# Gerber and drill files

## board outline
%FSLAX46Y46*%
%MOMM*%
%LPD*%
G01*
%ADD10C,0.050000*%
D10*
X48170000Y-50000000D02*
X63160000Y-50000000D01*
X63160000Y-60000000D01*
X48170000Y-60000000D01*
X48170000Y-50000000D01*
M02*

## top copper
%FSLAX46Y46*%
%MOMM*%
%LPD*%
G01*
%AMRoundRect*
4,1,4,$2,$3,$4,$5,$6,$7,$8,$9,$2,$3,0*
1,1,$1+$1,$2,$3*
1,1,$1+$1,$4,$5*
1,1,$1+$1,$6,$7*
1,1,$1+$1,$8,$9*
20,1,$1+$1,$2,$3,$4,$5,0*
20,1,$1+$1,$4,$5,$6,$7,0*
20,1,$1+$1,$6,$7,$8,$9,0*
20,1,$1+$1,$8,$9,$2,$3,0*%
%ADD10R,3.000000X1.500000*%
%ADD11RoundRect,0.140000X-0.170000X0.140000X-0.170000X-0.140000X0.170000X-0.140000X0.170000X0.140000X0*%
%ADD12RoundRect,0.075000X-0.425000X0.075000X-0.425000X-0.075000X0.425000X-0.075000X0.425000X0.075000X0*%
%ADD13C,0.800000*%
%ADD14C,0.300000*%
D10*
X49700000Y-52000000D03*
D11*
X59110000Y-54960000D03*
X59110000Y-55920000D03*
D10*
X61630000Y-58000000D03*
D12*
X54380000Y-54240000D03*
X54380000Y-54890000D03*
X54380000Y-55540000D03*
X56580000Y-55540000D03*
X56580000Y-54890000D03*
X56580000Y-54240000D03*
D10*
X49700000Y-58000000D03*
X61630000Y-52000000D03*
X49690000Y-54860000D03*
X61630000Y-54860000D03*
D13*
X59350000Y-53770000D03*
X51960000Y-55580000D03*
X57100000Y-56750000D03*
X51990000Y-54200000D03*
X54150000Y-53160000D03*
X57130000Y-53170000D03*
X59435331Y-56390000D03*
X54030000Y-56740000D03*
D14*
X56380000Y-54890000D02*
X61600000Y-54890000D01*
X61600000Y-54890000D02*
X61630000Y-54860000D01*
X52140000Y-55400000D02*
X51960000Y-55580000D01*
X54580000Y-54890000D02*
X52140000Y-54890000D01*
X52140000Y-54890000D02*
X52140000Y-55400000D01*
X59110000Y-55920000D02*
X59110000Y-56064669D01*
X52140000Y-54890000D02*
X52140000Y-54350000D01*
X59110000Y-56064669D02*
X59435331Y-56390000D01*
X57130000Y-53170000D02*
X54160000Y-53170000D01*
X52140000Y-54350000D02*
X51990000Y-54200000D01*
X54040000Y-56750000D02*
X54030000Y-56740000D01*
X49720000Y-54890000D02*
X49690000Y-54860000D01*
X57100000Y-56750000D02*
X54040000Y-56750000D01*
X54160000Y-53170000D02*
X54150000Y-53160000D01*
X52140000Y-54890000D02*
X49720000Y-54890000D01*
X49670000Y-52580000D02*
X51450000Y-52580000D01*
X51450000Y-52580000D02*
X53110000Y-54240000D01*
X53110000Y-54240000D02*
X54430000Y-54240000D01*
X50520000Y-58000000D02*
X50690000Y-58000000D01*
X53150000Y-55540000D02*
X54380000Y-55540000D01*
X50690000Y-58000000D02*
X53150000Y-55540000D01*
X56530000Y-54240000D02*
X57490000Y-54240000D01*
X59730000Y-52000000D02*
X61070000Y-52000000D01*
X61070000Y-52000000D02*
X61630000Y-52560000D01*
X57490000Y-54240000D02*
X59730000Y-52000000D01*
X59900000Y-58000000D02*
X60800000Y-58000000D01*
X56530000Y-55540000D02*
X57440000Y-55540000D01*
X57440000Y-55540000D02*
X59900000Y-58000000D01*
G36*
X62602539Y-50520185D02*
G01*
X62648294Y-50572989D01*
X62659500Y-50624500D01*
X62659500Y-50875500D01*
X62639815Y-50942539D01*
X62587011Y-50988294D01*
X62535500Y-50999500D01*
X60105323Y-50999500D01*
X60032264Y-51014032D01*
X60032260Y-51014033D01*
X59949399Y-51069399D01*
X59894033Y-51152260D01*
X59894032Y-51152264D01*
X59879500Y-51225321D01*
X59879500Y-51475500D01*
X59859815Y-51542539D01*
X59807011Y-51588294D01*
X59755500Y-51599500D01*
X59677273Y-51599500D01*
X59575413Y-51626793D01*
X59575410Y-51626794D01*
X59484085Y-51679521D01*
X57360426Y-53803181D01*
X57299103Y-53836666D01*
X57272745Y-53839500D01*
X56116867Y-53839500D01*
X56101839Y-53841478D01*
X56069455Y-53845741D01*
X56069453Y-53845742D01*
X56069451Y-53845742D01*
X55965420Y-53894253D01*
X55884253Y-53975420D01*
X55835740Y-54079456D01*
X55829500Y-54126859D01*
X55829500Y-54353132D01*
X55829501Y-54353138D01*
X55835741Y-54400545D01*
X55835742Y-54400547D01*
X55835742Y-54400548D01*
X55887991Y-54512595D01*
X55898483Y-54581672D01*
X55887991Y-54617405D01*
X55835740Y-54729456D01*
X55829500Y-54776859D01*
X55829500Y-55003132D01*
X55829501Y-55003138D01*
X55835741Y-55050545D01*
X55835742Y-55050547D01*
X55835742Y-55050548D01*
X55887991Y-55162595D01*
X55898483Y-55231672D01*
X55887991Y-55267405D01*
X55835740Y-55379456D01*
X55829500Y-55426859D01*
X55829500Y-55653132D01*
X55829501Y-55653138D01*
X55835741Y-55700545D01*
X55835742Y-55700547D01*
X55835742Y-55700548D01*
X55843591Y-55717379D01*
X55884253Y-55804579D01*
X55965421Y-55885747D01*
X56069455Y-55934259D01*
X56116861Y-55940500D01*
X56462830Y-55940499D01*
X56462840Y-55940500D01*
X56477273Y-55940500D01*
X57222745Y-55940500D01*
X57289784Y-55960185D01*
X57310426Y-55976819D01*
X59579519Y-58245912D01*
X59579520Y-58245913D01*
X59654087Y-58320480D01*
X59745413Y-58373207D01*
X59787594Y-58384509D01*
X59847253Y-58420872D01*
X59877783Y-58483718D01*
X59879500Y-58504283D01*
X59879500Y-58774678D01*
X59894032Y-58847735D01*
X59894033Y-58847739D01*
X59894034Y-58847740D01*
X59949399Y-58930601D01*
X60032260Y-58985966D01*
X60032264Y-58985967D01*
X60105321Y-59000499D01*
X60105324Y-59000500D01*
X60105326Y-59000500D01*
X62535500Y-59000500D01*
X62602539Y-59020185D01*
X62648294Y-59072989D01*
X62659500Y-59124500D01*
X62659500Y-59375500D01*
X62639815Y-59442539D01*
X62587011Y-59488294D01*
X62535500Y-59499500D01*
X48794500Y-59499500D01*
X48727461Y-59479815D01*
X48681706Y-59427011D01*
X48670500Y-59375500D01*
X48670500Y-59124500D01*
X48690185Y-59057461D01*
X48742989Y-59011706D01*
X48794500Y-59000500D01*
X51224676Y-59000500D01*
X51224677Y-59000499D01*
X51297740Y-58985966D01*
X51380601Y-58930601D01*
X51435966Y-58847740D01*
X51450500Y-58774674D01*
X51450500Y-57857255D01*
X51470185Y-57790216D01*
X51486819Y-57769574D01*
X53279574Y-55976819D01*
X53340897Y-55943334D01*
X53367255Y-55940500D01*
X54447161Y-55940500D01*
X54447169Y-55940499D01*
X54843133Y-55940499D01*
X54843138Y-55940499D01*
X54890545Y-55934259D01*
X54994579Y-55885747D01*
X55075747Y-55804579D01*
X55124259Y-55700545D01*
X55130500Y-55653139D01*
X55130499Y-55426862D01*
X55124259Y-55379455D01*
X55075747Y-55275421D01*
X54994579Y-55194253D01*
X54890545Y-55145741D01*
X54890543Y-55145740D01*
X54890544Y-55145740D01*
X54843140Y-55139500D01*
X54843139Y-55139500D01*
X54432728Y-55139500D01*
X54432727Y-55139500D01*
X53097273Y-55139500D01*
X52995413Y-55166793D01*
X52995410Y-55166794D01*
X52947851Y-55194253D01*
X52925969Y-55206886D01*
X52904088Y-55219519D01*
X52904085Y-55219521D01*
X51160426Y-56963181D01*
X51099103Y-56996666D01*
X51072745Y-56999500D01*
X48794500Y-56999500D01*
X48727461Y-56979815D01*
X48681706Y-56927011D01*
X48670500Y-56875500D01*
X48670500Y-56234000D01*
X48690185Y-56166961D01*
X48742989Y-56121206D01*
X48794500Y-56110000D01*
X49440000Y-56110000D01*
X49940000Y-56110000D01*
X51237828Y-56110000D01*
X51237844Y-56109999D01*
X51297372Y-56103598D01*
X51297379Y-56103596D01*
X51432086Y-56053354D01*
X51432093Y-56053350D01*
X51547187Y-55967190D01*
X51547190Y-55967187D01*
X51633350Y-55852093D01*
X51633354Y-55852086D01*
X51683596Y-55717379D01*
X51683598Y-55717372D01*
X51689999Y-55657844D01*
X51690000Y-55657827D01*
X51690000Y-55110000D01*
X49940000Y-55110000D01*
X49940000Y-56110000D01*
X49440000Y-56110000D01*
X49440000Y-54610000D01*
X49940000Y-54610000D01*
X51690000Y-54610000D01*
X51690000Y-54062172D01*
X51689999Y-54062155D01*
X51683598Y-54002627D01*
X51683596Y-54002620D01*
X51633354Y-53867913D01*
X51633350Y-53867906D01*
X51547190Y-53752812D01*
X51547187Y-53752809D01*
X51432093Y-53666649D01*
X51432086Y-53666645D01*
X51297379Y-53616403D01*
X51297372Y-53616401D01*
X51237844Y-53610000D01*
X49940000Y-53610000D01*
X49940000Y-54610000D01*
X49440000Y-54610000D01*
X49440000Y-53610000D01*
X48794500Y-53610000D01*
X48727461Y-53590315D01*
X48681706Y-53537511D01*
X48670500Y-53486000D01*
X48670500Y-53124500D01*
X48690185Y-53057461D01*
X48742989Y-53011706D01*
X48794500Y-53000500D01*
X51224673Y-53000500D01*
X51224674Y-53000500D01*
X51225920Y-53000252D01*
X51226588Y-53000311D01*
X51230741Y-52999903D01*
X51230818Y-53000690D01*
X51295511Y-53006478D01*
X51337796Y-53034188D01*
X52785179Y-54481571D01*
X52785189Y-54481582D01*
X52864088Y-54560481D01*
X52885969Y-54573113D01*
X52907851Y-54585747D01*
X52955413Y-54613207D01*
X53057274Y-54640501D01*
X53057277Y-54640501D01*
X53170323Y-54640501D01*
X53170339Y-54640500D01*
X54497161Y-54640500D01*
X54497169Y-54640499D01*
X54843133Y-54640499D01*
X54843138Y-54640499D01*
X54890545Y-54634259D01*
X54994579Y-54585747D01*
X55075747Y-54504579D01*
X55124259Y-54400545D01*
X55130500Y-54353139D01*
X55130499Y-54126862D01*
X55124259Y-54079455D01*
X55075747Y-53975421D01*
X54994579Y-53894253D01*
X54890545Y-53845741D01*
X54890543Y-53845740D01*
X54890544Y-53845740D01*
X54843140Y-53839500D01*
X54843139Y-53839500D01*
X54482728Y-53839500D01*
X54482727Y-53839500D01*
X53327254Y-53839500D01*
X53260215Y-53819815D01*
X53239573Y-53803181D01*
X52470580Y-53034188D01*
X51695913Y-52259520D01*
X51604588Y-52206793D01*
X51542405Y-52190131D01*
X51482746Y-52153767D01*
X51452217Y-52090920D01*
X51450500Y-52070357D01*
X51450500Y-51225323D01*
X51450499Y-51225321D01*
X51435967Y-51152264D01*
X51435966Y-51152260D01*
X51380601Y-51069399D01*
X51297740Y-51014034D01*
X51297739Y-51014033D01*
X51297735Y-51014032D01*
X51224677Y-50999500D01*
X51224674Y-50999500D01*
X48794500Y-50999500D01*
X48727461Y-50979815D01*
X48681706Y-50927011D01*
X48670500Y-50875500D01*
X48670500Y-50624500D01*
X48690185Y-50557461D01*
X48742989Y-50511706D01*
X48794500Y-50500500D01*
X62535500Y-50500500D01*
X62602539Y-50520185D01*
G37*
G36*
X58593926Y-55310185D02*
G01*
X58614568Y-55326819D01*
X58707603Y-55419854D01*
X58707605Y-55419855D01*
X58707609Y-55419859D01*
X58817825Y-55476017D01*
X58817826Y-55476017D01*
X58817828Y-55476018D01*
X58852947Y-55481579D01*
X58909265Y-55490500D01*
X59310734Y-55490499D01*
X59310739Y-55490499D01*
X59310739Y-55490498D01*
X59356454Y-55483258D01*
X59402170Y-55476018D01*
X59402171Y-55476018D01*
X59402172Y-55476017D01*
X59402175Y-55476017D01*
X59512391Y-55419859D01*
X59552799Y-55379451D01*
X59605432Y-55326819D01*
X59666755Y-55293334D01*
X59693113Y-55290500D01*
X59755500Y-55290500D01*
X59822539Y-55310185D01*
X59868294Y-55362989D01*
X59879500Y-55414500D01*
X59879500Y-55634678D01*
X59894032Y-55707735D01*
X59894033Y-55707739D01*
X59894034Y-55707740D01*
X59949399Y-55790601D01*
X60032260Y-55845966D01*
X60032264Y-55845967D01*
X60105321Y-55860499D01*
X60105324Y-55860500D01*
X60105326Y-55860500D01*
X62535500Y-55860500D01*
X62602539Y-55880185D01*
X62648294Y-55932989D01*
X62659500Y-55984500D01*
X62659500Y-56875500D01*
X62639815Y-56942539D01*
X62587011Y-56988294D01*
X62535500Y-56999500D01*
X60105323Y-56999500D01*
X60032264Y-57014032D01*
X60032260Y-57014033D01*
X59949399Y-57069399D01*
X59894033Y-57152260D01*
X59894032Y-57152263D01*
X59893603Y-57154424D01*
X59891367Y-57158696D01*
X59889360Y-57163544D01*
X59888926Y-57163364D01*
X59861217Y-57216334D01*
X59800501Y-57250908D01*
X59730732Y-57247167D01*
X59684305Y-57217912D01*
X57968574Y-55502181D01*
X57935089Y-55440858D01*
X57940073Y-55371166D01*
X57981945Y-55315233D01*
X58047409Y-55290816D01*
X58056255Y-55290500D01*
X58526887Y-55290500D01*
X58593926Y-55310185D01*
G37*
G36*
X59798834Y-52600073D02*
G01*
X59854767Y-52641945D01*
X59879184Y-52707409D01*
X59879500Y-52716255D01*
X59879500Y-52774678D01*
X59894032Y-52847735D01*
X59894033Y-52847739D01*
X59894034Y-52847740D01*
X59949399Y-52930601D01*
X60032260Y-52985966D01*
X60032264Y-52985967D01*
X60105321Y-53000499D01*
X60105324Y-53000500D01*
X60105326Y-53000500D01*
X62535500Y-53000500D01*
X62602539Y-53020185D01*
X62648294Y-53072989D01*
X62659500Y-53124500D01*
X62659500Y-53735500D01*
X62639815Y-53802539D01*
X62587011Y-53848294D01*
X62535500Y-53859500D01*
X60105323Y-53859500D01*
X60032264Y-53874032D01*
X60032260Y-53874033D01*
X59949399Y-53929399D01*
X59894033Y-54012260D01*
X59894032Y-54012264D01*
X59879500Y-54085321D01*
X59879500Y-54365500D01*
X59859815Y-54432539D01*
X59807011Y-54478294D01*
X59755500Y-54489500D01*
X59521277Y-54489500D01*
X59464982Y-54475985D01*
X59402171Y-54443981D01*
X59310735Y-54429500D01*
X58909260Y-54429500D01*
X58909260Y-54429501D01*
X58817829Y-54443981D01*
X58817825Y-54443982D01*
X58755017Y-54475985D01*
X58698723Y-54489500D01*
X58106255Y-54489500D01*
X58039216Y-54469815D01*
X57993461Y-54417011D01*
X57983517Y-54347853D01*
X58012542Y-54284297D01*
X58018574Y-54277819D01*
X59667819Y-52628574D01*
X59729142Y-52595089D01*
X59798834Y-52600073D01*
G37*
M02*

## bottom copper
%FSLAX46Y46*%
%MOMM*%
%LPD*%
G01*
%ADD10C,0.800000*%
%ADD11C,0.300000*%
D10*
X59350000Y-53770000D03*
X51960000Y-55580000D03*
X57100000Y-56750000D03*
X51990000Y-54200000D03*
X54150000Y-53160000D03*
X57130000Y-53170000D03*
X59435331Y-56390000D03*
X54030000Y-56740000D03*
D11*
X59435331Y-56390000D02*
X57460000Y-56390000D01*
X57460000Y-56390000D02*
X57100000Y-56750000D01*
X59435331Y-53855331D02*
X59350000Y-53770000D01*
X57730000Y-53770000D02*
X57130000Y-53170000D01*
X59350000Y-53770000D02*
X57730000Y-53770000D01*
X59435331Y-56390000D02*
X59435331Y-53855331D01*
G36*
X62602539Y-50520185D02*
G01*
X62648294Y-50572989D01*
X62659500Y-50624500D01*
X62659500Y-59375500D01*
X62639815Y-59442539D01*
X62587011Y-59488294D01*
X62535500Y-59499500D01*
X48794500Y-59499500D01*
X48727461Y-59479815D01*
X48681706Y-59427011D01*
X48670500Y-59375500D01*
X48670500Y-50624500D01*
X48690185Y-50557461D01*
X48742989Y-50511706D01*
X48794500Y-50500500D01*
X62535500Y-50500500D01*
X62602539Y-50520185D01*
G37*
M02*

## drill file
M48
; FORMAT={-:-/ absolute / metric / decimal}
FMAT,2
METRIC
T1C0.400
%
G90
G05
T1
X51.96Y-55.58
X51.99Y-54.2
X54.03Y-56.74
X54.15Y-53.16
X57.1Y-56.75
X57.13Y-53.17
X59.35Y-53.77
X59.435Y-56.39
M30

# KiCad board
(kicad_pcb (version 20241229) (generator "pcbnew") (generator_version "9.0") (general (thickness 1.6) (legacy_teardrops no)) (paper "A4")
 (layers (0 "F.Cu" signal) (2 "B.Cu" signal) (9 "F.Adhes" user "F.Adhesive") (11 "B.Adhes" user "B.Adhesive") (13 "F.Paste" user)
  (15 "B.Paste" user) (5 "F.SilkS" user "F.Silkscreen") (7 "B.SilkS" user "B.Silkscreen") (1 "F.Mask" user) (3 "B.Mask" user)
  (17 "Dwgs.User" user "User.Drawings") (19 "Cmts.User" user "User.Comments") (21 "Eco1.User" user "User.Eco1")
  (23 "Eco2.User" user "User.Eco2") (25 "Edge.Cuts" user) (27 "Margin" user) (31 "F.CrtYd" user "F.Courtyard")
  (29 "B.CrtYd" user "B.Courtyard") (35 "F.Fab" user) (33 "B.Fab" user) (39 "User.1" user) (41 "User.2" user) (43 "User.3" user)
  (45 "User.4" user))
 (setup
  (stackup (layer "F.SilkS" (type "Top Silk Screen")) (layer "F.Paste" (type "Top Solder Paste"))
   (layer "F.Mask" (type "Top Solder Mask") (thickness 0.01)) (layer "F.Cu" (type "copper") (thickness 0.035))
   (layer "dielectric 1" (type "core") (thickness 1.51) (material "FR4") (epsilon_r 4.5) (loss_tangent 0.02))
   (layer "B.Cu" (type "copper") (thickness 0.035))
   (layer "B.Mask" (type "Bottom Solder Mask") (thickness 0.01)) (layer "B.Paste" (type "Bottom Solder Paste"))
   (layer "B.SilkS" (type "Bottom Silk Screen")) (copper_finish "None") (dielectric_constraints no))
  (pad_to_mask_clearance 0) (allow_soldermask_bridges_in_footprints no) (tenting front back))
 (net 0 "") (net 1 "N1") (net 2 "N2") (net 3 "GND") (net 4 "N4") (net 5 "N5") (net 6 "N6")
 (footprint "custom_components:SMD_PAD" (layer "F.Cu") (at 49.7 52)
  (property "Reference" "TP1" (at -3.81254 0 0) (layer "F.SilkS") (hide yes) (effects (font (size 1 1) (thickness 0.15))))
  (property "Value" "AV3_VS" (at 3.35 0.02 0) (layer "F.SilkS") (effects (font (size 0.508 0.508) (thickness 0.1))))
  (pad "1" smd rect (at 0 0) (size 3 1.5) (layers "F.Cu" "F.Mask") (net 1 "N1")))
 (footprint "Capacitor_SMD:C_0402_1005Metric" (layer "F.Cu") (at 59.11 55.44 -90)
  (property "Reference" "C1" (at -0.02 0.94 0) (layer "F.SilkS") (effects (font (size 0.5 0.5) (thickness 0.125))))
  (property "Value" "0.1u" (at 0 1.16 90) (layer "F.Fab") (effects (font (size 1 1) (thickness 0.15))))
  (pad "1" smd roundrect (at -0.48 0 270) (size 0.56 0.62) (layers "F.Cu" "F.Mask" "F.Paste") (roundrect_rratio 0.25) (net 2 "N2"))
  (pad "2" smd roundrect (at 0.48 0 270) (size 0.56 0.62) (layers "F.Cu" "F.Mask" "F.Paste") (roundrect_rratio 0.25) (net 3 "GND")))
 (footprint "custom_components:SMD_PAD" (layer "F.Cu") (at 61.63 58 180)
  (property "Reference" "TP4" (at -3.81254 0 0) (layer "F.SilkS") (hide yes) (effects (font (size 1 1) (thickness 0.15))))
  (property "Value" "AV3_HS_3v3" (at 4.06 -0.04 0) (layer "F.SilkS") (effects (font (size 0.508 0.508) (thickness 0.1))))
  (pad "1" smd rect (at 0 0 180) (size 3 1.5) (layers "F.Cu" "F.Mask") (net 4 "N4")))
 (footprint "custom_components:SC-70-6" (layer "F.Cu") (at 55.48 54.89)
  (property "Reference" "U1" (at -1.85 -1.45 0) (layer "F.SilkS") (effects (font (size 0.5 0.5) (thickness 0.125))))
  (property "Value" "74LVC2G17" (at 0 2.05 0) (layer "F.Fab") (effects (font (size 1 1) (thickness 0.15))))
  (pad "1" smd roundrect (at -1.1 -0.65 270) (size 0.3 1) (layers "F.Cu" "F.Mask" "F.Paste") (roundrect_rratio 0.25) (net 1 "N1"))
  (pad "2" smd roundrect (at -1.1 0 270) (size 0.3 1) (layers "F.Cu" "F.Mask" "F.Paste") (roundrect_rratio 0.25) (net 3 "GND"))
  (pad "3" smd roundrect (at -1.1 0.65 270) (size 0.3 1) (layers "F.Cu" "F.Mask" "F.Paste") (roundrect_rratio 0.25) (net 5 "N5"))
  (pad "4" smd roundrect (at 1.1 0.65 270) (size 0.3 1) (layers "F.Cu" "F.Mask" "F.Paste") (roundrect_rratio 0.25) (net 4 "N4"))
  (pad "5" smd roundrect (at 1.1 0 270) (size 0.3 1) (layers "F.Cu" "F.Mask" "F.Paste") (roundrect_rratio 0.25) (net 2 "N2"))
  (pad "6" smd roundrect (at 1.1 -0.65 270) (size 0.3 1) (layers "F.Cu" "F.Mask" "F.Paste") (roundrect_rratio 0.25) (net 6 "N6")))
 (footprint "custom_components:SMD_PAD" (layer "F.Cu") (at 49.7 58)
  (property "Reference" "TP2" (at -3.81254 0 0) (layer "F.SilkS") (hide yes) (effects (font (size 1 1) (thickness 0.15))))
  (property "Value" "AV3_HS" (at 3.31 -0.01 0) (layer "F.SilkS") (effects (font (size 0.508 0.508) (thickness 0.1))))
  (pad "1" smd rect (at 0 0) (size 3 1.5) (layers "F.Cu" "F.Mask") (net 5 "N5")))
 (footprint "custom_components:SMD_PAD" (layer "F.Cu") (at 61.63 52 180)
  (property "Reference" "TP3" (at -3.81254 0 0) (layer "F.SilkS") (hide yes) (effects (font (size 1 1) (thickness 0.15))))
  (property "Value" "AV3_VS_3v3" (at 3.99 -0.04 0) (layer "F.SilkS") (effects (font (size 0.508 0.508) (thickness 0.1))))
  (pad "1" smd rect (at 0 0 180) (size 3 1.5) (layers "F.Cu" "F.Mask") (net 6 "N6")))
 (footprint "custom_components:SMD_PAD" (layer "F.Cu") (at 49.69 54.86)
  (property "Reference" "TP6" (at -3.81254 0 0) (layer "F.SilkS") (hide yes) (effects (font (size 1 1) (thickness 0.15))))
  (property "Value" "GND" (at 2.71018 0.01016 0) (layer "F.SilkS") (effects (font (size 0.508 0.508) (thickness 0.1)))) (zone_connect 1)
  (pad "1" smd rect (at 0 0) (size 3 1.5) (layers "F.Cu" "F.Mask") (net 3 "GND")))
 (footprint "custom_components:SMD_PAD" (layer "F.Cu") (at 61.63 54.86 180)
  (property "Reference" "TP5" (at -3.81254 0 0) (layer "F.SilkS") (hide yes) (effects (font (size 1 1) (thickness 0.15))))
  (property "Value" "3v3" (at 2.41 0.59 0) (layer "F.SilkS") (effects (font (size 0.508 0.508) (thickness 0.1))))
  (pad "1" smd rect (at 0 0 180) (size 3 1.5) (layers "F.Cu" "F.Mask") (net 2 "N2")))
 (gr_rect (start 48.17 50) (end 63.16 60) (stroke (width 0.05) (type solid)) (fill no) (layer "Edge.Cuts"))
 (segment (start 56.38 54.89) (end 61.6 54.89) (width 0.3) (layer "F.Cu") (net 2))
 (segment (start 61.6 54.89) (end 61.63 54.86) (width 0.3) (layer "F.Cu") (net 2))
 (segment (start 52.14 55.4) (end 51.96 55.58) (width 0.3) (layer "F.Cu") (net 3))
 (segment (start 54.58 54.89) (end 52.14 54.89) (width 0.3) (layer "F.Cu") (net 3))
 (segment (start 52.14 54.89) (end 52.14 55.4) (width 0.3) (layer "F.Cu") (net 3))
 (segment (start 59.11 55.92) (end 59.11 56.064669) (width 0.3) (layer "F.Cu") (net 3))
 (segment (start 52.14 54.89) (end 52.14 54.35) (width 0.3) (layer "F.Cu") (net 3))
 (segment (start 59.11 56.064669) (end 59.435331 56.39) (width 0.3) (layer "F.Cu") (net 3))
 (segment (start 57.13 53.17) (end 54.16 53.17) (width 0.3) (layer "F.Cu") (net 3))
 (segment (start 52.14 54.35) (end 51.99 54.2) (width 0.3) (layer "F.Cu") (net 3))
 (segment (start 54.04 56.75) (end 54.03 56.74) (width 0.3) (layer "F.Cu") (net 3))
 (segment (start 49.72 54.89) (end 49.69 54.86) (width 0.3) (layer "F.Cu") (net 3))
 (segment (start 57.1 56.75) (end 54.04 56.75) (width 0.3) (layer "F.Cu") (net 3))
 (segment (start 54.16 53.17) (end 54.15 53.16) (width 0.3) (layer "F.Cu") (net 3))
 (segment (start 52.14 54.89) (end 49.72 54.89) (width 0.3) (layer "F.Cu") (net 3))
 (via (at 59.35 53.77) (size 0.8) (drill 0.4) (layers "F.Cu" "B.Cu") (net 3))
 (via (at 51.96 55.58) (size 0.8) (drill 0.4) (layers "F.Cu" "B.Cu") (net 3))
 (via (at 57.1 56.75) (size 0.8) (drill 0.4) (layers "F.Cu" "B.Cu") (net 3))
 (via (at 51.99 54.2) (size 0.8) (drill 0.4) (layers "F.Cu" "B.Cu") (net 3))
 (via (at 54.15 53.16) (size 0.8) (drill 0.4) (layers "F.Cu" "B.Cu") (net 3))
 (via (at 57.13 53.17) (size 0.8) (drill 0.4) (layers "F.Cu" "B.Cu") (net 3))
 (via (at 59.435331 56.39) (size 0.8) (drill 0.4) (layers "F.Cu" "B.Cu") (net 3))
 (via (at 54.03 56.74) (size 0.8) (drill 0.4) (layers "F.Cu" "B.Cu") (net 3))
 (segment (start 59.435331 56.39) (end 57.46 56.39) (width 0.3) (layer "B.Cu") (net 3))
 (segment (start 57.46 56.39) (end 57.1 56.75) (width 0.3) (layer "B.Cu") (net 3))
 (segment (start 59.435331 53.855331) (end 59.35 53.77) (width 0.3) (layer "B.Cu") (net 3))
 (segment (start 57.73 53.77) (end 57.13 53.17) (width 0.3) (layer "B.Cu") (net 3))
 (segment (start 59.35 53.77) (end 57.73 53.77) (width 0.3) (layer "B.Cu") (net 3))
 (segment (start 59.435331 56.39) (end 59.435331 53.855331) (width 0.3) (layer "B.Cu") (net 3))
 (segment (start 49.67 52.58) (end 51.45 52.58) (width 0.3) (layer "F.Cu") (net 1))
 (segment (start 51.45 52.58) (end 53.11 54.24) (width 0.3) (layer "F.Cu") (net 1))
 (segment (start 53.11 54.24) (end 54.43 54.24) (width 0.3) (layer "F.Cu") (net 1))
 (segment (start 50.52 58) (end 50.69 58) (width 0.3) (layer "F.Cu") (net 5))
 (segment (start 53.15 55.54) (end 54.38 55.54) (width 0.3) (layer "F.Cu") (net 5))
 (segment (start 50.69 58) (end 53.15 55.54) (width 0.3) (layer "F.Cu") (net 5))
 (segment (start 56.53 54.24) (end 57.49 54.24) (width 0.3) (layer "F.Cu") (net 6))
 (segment (start 59.73 52) (end 61.07 52) (width 0.3) (layer "F.Cu") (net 6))
 (segment (start 61.07 52) (end 61.63 52.56) (width 0.3) (layer "F.Cu") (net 6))
 (segment (start 57.49 54.24) (end 59.73 52) (width 0.3) (layer "F.Cu") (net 6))
 (segment (start 59.9 58) (end 60.8 58) (width 0.3) (layer "F.Cu") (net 4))
 (segment (start 56.53 55.54) (end 57.44 55.54) (width 0.3) (layer "F.Cu") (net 4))
 (segment (start 57.44 55.54) (end 59.9 58) (width 0.3) (layer "F.Cu") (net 4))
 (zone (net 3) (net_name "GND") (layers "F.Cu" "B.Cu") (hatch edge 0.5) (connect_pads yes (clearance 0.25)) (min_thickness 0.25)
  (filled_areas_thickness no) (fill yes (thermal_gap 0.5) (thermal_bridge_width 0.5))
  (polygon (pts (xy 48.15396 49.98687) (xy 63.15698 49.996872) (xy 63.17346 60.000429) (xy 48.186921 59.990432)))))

